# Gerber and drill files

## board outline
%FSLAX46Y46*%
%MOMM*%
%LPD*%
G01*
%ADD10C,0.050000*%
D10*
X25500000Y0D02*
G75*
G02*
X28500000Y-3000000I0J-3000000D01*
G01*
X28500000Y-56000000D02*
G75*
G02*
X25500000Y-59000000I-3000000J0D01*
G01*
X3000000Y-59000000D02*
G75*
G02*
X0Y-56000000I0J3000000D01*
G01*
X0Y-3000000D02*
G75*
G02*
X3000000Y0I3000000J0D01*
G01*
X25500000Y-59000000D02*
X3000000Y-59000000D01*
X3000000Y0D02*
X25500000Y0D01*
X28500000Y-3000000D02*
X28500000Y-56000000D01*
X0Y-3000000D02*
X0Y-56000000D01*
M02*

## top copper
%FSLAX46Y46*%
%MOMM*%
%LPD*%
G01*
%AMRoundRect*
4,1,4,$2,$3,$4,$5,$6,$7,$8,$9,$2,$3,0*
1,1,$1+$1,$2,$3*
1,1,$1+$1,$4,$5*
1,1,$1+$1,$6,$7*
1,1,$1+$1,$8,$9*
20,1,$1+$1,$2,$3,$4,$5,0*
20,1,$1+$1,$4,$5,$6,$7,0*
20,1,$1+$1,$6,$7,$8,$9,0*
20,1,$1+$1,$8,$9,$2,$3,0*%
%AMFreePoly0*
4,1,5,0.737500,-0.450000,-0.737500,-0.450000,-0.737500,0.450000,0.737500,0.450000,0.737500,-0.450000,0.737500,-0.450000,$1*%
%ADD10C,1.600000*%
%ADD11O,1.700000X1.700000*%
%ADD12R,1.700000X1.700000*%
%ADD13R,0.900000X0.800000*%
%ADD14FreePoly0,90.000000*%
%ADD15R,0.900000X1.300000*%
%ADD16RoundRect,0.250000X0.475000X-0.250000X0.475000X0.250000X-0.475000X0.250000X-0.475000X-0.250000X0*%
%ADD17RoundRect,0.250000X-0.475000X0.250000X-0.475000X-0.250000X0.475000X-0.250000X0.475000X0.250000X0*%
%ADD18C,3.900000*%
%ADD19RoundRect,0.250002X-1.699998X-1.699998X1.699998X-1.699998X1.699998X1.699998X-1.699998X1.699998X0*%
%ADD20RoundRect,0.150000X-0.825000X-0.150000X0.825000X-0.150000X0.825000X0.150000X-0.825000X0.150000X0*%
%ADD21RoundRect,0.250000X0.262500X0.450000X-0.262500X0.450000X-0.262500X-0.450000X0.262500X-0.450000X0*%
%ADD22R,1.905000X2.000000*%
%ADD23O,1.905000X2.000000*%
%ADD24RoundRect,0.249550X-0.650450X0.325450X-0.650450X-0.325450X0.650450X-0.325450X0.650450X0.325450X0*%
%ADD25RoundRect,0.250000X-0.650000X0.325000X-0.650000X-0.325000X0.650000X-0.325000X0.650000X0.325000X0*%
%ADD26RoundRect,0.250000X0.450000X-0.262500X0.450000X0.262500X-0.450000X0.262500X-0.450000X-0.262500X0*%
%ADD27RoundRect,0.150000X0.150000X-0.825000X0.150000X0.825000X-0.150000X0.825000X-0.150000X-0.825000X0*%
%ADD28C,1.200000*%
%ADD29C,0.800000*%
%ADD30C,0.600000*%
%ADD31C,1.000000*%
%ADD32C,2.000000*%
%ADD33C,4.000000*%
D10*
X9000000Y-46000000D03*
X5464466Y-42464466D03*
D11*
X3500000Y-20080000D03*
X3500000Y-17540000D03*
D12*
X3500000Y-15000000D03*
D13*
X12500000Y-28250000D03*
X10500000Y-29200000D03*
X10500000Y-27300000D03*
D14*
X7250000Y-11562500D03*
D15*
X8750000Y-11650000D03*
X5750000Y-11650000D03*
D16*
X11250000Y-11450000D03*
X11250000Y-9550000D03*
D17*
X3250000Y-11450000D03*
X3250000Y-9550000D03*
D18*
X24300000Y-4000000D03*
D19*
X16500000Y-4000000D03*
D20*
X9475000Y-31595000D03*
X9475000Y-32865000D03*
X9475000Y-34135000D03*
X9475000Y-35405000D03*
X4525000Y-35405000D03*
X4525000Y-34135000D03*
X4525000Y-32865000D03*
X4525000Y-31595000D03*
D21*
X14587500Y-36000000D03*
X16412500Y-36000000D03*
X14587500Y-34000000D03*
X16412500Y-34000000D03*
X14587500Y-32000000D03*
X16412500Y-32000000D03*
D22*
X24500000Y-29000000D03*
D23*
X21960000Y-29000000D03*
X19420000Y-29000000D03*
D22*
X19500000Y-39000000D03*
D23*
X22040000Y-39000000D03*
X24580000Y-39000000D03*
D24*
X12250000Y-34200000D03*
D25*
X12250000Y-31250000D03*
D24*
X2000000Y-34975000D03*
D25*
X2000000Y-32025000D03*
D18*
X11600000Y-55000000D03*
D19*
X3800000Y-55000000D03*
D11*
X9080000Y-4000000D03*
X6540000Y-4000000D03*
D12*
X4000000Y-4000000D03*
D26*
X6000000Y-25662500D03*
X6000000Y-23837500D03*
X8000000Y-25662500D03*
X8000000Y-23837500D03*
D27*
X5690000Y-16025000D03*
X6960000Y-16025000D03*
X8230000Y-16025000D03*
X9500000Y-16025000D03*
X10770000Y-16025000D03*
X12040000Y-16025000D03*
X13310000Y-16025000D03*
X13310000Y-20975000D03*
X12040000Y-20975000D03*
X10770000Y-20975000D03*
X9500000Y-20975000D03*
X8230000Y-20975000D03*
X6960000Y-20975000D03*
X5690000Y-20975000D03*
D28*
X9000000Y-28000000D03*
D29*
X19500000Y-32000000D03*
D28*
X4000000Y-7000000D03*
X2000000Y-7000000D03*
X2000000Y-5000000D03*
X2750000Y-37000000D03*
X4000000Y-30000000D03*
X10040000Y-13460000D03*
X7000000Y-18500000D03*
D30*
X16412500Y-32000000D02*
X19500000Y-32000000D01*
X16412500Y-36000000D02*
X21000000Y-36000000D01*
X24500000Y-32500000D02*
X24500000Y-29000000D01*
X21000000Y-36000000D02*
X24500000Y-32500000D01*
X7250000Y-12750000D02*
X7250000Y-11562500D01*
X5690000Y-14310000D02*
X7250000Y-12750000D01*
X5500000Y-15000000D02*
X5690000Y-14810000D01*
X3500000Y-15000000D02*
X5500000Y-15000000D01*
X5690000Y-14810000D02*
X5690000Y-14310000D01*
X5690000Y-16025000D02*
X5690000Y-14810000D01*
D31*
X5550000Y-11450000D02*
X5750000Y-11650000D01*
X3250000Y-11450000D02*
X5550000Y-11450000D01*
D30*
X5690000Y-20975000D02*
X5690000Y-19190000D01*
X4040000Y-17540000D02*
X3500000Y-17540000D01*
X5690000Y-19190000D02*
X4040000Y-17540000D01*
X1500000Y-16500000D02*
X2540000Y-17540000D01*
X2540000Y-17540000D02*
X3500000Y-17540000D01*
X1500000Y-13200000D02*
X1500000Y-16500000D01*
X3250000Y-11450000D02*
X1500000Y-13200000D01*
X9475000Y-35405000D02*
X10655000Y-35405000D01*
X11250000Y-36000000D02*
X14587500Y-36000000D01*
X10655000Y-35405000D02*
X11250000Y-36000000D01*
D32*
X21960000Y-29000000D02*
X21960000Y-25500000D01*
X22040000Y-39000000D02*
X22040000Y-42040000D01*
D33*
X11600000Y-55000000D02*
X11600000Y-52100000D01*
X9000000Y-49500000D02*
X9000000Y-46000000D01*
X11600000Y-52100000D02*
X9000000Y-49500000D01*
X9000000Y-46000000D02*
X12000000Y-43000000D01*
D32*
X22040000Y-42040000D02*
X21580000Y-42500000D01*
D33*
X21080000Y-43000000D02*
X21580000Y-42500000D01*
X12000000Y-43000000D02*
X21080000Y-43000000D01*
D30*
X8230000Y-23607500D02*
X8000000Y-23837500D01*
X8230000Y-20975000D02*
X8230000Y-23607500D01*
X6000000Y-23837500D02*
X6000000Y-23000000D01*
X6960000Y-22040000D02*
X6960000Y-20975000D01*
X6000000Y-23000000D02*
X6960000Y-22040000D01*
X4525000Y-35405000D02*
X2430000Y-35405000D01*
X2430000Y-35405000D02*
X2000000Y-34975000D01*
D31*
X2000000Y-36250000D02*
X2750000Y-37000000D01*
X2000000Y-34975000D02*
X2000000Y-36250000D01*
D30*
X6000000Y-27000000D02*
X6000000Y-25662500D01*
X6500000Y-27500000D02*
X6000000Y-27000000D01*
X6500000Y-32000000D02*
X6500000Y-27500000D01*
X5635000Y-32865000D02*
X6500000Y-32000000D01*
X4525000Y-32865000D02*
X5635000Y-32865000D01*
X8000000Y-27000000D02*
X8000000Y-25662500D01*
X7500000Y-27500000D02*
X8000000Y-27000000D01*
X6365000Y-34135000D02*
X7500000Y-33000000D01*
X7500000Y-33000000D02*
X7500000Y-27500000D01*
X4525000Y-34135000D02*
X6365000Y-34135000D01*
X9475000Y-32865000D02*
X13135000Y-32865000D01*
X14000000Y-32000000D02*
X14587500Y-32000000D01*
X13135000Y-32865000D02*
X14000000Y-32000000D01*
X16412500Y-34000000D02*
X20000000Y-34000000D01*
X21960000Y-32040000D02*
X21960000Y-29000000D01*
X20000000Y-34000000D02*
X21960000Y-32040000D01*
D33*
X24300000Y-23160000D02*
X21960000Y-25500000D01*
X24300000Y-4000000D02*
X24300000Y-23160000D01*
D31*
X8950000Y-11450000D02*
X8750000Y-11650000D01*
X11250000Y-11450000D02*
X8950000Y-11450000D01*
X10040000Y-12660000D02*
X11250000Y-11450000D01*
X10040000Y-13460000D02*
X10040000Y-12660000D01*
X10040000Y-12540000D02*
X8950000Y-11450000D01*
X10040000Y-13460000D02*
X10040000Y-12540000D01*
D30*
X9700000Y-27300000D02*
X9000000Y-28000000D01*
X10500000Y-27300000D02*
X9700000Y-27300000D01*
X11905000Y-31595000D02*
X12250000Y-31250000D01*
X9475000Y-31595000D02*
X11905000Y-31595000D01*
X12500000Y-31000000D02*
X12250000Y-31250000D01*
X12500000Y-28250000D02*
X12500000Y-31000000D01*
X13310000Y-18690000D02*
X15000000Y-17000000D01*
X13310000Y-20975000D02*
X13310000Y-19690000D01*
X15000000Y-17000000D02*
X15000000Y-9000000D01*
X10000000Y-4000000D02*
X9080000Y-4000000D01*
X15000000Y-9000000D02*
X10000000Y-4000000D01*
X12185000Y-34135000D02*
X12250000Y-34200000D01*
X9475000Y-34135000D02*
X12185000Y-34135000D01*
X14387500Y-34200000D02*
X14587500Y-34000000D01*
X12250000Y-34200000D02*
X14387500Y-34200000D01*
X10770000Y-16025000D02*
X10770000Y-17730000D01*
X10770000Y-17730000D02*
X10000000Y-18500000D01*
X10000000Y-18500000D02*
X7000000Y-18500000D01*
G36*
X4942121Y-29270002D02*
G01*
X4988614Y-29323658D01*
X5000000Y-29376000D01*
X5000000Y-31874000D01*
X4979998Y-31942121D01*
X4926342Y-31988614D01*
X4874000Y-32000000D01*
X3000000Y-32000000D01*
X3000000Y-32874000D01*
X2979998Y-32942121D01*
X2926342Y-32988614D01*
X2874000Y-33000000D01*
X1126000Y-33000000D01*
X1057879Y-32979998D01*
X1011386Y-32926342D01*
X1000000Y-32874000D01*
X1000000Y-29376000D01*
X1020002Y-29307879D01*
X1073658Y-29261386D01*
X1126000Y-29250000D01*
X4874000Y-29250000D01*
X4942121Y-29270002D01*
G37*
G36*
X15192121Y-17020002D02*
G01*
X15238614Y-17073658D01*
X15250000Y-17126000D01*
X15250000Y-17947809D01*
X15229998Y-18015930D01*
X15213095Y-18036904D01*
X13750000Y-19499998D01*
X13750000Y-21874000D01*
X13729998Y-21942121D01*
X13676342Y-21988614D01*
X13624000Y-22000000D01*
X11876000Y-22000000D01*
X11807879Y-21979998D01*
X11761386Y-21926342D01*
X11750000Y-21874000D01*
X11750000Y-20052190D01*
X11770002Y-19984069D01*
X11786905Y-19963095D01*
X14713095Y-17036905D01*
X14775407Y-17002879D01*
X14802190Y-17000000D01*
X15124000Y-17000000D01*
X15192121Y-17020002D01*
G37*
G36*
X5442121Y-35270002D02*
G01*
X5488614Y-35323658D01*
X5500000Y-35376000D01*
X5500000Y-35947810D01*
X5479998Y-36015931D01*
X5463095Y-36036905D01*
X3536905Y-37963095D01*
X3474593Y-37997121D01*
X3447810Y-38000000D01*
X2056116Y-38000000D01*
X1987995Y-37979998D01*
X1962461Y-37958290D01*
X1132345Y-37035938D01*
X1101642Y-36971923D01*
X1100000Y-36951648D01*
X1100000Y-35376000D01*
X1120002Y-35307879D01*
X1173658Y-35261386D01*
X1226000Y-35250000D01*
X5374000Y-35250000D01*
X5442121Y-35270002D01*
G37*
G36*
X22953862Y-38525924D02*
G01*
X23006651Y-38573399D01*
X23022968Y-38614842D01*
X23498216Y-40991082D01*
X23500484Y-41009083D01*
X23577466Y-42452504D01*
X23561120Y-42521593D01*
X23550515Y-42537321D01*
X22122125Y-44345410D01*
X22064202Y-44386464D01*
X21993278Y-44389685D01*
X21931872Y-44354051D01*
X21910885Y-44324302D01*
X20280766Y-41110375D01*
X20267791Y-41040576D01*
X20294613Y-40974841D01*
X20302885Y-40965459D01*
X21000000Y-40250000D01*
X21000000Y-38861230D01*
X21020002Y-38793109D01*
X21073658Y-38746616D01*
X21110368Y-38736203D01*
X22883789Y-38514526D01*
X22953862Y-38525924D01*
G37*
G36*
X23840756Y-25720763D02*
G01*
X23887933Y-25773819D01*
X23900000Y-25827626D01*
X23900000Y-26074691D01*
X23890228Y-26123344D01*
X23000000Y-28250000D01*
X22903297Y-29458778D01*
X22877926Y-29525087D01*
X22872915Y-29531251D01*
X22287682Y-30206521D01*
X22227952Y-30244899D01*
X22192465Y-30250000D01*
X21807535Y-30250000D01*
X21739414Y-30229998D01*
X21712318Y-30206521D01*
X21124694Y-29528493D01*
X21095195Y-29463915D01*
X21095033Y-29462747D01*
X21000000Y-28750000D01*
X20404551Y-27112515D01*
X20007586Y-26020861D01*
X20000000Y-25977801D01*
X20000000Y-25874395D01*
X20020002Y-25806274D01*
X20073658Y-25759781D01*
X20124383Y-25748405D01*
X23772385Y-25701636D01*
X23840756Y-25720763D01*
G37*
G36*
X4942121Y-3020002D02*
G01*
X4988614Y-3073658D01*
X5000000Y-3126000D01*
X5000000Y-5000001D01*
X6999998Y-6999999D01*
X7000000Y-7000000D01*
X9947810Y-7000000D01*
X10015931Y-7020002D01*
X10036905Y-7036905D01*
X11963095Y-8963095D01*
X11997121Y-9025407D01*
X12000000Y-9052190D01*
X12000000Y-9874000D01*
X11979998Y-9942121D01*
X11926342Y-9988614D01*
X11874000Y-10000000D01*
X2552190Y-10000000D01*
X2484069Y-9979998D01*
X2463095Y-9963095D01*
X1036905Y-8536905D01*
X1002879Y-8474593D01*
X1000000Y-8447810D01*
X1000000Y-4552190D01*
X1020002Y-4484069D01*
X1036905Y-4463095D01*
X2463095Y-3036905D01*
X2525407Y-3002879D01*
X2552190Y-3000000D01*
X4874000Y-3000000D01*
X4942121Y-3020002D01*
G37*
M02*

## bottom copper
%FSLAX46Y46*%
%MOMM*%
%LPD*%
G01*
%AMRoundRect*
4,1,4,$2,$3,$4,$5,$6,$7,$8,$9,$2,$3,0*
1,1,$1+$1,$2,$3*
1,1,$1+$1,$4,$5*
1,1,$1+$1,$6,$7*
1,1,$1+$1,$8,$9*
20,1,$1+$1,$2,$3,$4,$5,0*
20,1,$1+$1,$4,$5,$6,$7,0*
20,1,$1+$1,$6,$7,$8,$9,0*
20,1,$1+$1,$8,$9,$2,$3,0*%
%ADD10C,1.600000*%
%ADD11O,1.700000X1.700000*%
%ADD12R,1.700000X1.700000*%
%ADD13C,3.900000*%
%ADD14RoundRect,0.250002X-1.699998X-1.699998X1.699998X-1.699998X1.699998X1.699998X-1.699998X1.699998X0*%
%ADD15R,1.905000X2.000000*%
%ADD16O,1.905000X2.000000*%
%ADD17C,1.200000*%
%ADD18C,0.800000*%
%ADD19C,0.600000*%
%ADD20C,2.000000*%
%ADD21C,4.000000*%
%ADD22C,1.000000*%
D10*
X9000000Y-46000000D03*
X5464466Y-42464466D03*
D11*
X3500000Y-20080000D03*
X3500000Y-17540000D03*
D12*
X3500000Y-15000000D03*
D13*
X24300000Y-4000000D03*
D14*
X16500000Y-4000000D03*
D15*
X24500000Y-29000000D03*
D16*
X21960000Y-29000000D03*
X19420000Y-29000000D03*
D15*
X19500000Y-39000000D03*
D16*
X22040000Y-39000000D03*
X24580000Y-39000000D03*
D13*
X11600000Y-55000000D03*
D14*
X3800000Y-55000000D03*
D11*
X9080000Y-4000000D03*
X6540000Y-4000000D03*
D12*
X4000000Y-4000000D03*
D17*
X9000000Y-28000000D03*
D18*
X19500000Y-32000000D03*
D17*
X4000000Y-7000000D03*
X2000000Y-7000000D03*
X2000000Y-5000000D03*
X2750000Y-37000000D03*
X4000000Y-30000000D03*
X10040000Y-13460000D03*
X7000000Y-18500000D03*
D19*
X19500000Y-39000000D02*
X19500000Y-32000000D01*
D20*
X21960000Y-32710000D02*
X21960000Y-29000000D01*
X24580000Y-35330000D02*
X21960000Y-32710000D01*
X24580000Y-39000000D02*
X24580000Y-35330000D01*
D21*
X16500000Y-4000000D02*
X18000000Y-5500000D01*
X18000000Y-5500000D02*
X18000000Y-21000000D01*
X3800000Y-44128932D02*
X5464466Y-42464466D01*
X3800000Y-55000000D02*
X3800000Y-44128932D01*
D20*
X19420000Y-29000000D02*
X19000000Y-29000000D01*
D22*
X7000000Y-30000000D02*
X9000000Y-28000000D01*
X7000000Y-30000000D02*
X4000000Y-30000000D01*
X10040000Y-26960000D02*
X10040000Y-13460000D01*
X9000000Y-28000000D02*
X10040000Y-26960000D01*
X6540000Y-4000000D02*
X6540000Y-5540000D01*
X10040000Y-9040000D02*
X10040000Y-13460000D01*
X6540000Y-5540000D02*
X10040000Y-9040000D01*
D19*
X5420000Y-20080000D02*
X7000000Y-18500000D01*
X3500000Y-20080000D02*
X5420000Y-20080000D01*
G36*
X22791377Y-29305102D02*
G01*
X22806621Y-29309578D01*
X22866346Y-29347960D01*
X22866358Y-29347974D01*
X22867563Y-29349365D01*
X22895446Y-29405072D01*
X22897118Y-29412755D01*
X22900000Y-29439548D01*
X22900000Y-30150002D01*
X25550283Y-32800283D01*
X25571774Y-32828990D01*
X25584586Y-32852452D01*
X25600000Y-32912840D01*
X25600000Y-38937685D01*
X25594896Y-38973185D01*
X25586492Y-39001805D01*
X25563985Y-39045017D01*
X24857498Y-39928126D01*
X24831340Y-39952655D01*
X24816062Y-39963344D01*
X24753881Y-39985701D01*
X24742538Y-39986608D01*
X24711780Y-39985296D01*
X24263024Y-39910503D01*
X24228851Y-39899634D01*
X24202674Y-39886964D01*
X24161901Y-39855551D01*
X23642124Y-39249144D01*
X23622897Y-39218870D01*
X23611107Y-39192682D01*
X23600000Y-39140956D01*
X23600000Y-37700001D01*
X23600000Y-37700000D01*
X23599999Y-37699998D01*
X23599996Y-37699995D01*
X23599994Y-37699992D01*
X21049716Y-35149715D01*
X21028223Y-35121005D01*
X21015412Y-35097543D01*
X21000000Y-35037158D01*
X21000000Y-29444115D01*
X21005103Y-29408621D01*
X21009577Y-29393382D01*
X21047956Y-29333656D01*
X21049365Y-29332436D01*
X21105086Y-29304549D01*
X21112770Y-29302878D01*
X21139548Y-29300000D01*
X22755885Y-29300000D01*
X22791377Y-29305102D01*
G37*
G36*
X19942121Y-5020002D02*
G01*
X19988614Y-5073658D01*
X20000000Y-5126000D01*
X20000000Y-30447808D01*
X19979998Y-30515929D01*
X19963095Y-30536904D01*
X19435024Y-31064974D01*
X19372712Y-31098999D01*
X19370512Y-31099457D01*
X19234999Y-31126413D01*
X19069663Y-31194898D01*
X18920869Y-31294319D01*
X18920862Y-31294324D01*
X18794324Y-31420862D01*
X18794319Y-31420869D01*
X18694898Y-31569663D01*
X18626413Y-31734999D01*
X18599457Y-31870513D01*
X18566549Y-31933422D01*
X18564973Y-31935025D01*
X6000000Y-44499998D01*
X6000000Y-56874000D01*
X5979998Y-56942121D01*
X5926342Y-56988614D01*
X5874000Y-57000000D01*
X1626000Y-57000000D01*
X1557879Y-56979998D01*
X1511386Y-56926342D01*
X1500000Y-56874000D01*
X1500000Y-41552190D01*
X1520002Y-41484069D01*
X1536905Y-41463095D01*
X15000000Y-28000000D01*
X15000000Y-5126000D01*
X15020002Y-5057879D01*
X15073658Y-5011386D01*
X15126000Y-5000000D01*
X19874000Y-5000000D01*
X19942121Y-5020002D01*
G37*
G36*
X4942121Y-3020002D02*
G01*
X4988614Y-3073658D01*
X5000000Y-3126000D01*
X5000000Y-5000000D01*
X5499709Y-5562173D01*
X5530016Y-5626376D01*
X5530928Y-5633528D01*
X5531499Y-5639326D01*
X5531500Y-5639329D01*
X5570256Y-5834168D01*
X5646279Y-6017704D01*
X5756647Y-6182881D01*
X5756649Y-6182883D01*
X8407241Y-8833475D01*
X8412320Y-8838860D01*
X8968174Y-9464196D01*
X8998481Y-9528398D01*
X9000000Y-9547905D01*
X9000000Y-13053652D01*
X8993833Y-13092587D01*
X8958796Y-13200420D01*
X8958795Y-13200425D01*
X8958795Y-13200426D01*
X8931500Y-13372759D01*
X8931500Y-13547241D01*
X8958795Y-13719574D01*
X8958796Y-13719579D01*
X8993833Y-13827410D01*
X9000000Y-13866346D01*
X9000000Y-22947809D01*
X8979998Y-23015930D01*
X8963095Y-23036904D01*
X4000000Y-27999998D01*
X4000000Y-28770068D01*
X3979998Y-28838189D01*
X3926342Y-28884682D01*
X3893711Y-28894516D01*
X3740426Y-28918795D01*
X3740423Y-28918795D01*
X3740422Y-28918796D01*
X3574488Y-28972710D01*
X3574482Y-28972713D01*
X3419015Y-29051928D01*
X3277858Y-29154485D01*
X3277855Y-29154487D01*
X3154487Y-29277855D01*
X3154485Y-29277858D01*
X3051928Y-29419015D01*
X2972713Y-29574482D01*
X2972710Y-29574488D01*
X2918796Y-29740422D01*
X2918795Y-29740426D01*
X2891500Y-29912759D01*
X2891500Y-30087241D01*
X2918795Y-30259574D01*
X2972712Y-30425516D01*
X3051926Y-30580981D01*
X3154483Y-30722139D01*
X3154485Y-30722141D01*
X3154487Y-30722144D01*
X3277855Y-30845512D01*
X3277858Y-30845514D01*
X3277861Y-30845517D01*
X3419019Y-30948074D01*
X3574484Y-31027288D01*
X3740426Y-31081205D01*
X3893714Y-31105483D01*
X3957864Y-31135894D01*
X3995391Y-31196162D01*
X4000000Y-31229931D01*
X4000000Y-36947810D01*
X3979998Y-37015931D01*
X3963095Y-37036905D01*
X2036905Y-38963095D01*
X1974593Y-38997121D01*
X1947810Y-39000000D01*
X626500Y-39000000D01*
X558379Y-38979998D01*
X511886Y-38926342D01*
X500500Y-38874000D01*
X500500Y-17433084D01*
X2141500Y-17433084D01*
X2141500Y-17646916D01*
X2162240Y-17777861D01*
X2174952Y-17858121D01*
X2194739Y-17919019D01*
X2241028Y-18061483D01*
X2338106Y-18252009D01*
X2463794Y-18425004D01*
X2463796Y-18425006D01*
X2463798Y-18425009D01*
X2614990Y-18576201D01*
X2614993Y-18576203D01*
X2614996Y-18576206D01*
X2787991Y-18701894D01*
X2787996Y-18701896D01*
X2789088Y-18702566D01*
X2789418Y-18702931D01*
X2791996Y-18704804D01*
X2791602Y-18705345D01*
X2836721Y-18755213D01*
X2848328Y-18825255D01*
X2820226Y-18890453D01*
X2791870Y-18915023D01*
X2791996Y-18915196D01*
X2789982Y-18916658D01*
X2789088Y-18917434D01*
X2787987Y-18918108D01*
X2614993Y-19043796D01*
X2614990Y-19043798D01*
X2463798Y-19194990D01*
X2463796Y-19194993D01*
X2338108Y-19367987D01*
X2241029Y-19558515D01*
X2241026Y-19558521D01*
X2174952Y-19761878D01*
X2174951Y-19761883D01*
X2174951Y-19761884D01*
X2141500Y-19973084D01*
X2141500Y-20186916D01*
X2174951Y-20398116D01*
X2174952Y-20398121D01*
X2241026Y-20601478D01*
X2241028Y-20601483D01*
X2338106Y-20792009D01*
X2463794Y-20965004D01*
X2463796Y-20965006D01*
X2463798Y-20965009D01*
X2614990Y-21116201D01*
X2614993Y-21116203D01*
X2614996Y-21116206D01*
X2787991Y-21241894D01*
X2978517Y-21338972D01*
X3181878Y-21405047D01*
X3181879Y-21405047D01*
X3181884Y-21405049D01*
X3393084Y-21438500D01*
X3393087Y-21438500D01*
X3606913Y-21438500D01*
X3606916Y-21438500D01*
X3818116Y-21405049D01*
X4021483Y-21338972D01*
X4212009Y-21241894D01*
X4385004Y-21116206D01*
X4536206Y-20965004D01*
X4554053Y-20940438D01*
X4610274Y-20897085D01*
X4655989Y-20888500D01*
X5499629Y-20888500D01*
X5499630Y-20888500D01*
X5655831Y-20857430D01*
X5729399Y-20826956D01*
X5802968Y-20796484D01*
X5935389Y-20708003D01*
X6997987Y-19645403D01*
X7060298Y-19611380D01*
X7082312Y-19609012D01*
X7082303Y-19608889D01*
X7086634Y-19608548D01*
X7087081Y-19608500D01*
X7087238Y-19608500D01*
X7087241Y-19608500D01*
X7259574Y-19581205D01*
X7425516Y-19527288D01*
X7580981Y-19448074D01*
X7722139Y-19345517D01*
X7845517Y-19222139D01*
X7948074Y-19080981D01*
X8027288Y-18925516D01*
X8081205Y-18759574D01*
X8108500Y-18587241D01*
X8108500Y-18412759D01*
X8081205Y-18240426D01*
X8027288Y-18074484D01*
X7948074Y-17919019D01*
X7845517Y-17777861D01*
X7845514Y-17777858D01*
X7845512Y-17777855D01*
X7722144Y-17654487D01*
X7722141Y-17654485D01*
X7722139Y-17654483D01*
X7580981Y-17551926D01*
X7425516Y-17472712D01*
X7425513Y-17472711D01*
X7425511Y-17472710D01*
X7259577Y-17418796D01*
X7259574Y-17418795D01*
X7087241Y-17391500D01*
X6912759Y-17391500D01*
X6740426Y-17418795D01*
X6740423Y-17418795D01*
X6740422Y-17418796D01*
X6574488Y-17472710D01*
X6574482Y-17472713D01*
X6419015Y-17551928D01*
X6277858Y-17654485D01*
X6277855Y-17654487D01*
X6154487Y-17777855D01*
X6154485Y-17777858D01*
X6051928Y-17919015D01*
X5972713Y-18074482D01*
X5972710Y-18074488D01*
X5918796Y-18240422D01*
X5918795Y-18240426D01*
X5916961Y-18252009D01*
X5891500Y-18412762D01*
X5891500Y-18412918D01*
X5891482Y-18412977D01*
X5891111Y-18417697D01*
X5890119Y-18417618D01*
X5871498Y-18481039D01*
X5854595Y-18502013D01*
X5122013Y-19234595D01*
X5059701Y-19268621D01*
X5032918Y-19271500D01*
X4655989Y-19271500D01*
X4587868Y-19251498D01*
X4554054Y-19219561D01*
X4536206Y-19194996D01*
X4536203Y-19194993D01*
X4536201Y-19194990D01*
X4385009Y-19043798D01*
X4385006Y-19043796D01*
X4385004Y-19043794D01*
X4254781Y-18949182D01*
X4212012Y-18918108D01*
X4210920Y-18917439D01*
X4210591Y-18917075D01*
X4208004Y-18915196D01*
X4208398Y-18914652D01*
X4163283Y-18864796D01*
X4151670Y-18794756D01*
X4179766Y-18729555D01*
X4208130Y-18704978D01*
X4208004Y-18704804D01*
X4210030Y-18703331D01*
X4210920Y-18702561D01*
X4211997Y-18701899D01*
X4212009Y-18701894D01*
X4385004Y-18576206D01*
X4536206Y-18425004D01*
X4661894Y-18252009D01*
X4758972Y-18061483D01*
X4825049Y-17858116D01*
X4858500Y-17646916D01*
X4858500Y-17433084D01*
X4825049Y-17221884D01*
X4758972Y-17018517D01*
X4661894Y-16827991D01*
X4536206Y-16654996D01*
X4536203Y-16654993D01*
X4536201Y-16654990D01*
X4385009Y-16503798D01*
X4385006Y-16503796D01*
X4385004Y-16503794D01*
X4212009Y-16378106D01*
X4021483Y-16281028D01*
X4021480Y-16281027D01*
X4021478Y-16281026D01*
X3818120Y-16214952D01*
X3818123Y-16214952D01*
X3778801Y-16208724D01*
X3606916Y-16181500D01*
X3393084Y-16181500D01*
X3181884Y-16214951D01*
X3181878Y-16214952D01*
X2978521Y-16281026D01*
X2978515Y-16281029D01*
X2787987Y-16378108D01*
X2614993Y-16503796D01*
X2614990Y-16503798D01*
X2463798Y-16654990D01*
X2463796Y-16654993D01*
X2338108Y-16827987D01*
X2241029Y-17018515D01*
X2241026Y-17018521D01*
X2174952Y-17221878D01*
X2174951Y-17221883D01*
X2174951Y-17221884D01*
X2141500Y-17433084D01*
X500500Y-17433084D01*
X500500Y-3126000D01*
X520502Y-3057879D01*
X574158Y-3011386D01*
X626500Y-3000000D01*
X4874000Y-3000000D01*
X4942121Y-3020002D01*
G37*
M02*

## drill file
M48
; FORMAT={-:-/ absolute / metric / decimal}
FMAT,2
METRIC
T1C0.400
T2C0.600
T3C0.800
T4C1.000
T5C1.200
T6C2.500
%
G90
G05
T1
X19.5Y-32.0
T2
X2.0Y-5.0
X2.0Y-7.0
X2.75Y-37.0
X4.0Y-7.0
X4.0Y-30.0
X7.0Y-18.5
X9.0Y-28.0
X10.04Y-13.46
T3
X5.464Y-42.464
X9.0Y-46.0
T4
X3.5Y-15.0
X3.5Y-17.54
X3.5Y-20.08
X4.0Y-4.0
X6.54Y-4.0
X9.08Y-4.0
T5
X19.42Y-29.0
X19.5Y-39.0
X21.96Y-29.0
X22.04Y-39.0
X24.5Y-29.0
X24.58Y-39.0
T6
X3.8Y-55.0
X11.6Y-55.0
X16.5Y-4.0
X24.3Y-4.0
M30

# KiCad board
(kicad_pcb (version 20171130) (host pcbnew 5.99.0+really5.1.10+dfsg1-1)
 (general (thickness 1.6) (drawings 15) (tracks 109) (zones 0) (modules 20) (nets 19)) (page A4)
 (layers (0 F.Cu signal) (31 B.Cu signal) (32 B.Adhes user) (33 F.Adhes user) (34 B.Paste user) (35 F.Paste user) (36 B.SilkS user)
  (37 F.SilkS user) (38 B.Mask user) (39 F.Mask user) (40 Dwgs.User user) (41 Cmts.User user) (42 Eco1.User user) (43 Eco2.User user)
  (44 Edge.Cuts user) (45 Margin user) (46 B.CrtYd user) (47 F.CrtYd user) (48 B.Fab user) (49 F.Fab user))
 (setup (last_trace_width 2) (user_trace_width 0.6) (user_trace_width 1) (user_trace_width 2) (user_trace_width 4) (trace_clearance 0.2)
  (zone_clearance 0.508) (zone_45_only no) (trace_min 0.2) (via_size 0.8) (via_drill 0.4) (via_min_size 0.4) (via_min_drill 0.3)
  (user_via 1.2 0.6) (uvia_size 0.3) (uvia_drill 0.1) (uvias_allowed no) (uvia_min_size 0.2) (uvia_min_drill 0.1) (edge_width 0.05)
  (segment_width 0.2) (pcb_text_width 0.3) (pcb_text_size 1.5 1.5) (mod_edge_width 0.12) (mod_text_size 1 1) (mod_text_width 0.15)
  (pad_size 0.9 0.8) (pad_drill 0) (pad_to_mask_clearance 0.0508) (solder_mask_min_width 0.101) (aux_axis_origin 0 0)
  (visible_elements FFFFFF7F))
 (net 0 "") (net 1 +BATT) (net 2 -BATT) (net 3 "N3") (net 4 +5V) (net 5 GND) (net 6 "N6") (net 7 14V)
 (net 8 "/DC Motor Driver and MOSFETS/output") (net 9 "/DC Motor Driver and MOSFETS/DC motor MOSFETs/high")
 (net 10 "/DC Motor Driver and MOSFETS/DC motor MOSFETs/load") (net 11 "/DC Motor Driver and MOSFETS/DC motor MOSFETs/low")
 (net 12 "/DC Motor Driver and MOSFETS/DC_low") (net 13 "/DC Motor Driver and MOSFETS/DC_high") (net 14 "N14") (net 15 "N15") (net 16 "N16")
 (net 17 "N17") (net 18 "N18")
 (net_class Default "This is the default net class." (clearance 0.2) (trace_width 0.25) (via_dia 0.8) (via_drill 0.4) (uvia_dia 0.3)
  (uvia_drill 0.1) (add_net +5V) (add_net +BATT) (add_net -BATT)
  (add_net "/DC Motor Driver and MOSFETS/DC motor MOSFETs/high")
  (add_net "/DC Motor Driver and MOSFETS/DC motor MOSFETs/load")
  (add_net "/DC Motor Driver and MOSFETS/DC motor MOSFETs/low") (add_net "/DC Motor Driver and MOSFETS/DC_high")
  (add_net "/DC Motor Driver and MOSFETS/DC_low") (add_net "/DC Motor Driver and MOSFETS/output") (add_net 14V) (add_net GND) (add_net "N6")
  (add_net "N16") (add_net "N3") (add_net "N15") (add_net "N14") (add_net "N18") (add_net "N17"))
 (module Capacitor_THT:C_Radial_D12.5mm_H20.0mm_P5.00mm (layer F.Cu) (at 9 46 135)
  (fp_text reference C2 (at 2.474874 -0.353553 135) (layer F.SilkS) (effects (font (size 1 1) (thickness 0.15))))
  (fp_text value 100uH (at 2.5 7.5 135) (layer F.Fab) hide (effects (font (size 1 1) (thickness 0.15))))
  (pad 1 thru_hole circle (at 0 0 135) (size 1.6 1.6) (drill 0.8) (layers *.Cu *.Mask) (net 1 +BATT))
  (pad 2 thru_hole circle (at 5 0 135) (size 1.6 1.6) (drill 0.8) (layers *.Cu *.Mask) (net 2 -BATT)))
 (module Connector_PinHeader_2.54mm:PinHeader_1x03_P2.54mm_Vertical (layer B.Cu) (at 3.5 15 180)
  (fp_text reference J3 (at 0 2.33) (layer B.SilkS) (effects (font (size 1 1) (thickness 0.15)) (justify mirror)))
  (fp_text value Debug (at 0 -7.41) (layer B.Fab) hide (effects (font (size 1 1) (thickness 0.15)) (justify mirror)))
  (pad 3 thru_hole oval (at 0 -5.08 180) (size 1.7 1.7) (drill 1) (layers *.Cu *.Mask) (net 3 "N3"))
  (pad 2 thru_hole oval (at 0 -2.54 180) (size 1.7 1.7) (drill 1) (layers *.Cu *.Mask) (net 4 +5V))
  (pad 1 thru_hole rect (at 0 0 180) (size 1.7 1.7) (drill 1) (layers *.Cu *.Mask) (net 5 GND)))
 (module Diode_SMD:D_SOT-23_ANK (layer F.Cu) (at 11.5 28.25)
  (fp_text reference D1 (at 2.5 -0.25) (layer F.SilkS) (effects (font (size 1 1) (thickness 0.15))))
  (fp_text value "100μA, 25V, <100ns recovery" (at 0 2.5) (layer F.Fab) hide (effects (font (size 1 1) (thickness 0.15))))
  (pad 1 smd rect (at 1 0) (size 0.9 0.8) (layers F.Cu F.Paste F.Mask) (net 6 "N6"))
  (pad "" smd rect (at -1 0.95) (size 0.9 0.8) (layers F.Cu F.Paste F.Mask))
  (pad 2 smd rect (at -1 -0.95) (size 0.9 0.8) (layers F.Cu F.Paste F.Mask) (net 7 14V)))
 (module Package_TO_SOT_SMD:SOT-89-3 (layer F.Cu) (at 7.25 10 90)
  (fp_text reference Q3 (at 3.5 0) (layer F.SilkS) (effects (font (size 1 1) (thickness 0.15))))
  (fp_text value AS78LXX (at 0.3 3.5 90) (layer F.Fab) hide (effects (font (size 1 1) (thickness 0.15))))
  (pad 2 smd custom (at -1.5625 0 90) (size 1.475 0.9) (layers F.Cu F.Paste F.Mask) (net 5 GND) (zone_connect 2)
   (options (clearance outline) (anchor rect)) (primitives))
  (pad 3 smd rect (at -1.65 1.5 90) (size 1.3 0.9) (layers F.Cu F.Paste F.Mask) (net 7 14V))
  (pad 1 smd rect (at -1.65 -1.5 90) (size 1.3 0.9) (layers F.Cu F.Paste F.Mask) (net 4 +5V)))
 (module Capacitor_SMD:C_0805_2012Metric (layer F.Cu) (at 11.25 10.5 90)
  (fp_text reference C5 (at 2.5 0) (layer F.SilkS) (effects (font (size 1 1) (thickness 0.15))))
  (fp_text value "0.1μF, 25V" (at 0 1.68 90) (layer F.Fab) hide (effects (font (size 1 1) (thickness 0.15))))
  (pad 1 smd roundrect (at -0.95 0 90) (size 1 1.45) (layers F.Cu F.Paste F.Mask) (roundrect_rratio 0.25) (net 7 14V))
  (pad 2 smd roundrect (at 0.95 0 90) (size 1 1.45) (layers F.Cu F.Paste F.Mask) (roundrect_rratio 0.25) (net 5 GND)))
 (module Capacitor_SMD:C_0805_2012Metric (layer F.Cu) (at 3.25 10.5 270)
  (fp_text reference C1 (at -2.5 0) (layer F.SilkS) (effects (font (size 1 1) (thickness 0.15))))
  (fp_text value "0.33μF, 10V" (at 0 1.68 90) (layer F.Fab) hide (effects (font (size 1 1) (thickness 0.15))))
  (pad 2 smd roundrect (at 0.95 0 270) (size 1 1.45) (layers F.Cu F.Paste F.Mask) (roundrect_rratio 0.25) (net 4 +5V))
  (pad 1 smd roundrect (at -0.95 0 270) (size 1 1.45) (layers F.Cu F.Paste F.Mask) (roundrect_rratio 0.25) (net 5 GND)))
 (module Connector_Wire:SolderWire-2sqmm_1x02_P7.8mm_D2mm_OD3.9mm (layer F.Cu) (at 16.5 4)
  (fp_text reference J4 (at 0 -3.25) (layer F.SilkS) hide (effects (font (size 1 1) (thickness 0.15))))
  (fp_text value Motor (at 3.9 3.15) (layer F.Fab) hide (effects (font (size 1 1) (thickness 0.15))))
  (pad 2 thru_hole circle (at 7.8 0) (size 3.9 3.9) (drill 2.5) (layers *.Cu *.Mask) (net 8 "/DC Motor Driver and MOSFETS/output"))
  (pad 1 thru_hole roundrect (at 0 0) (size 3.9 3.9) (drill 2.5) (layers *.Cu *.Mask) (roundrect_rratio 0.06410299999999999) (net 2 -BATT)))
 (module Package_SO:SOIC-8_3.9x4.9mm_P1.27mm (layer F.Cu) (at 7 33.5)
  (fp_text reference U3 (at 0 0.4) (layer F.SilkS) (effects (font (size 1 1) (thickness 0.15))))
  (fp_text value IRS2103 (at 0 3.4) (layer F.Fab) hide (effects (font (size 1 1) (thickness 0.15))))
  (pad 8 smd roundrect (at 2.475 -1.905) (size 1.95 0.6) (layers F.Cu F.Paste F.Mask) (roundrect_rratio 0.25) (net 6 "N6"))
  (pad 7 smd roundrect (at 2.475 -0.635) (size 1.95 0.6) (layers F.Cu F.Paste F.Mask) (roundrect_rratio 0.25)
   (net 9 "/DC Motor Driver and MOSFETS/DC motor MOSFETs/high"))
  (pad 6 smd roundrect (at 2.475 0.635) (size 1.95 0.6) (layers F.Cu F.Paste F.Mask) (roundrect_rratio 0.25)
   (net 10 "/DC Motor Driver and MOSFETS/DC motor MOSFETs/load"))
  (pad 5 smd roundrect (at 2.475 1.905) (size 1.95 0.6) (layers F.Cu F.Paste F.Mask) (roundrect_rratio 0.25)
   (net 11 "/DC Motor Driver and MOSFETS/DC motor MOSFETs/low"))
  (pad 4 smd roundrect (at -2.475 1.905) (size 1.95 0.6) (layers F.Cu F.Paste F.Mask) (roundrect_rratio 0.25) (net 5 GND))
  (pad 3 smd roundrect (at -2.475 0.635) (size 1.95 0.6) (layers F.Cu F.Paste F.Mask) (roundrect_rratio 0.25)
   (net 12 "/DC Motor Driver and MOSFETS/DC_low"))
  (pad 2 smd roundrect (at -2.475 -0.635) (size 1.95 0.6) (layers F.Cu F.Paste F.Mask) (roundrect_rratio 0.25)
   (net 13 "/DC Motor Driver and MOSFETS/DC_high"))
  (pad 1 smd roundrect (at -2.475 -1.905) (size 1.95 0.6) (layers F.Cu F.Paste F.Mask) (roundrect_rratio 0.25) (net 7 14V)))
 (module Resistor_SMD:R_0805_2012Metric (layer F.Cu) (at 15.5 36 180)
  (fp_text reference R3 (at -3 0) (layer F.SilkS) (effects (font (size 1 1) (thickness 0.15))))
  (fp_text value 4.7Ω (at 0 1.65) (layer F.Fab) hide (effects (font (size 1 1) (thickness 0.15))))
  (pad 2 smd roundrect (at 0.9125 0 180) (size 1.025 1.4) (layers F.Cu F.Paste F.Mask) (roundrect_rratio 0.243902)
   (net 11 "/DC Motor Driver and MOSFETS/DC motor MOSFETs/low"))
  (pad 1 smd roundrect (at -0.9125 0 180) (size 1.025 1.4) (layers F.Cu F.Paste F.Mask) (roundrect_rratio 0.243902) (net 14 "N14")))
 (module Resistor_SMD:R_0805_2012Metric (layer F.Cu) (at 15.5 34 180)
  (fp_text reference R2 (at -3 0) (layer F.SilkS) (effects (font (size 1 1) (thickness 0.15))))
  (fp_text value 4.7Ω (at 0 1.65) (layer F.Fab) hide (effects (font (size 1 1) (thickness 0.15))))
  (pad 2 smd roundrect (at 0.9125 0 180) (size 1.025 1.4) (layers F.Cu F.Paste F.Mask) (roundrect_rratio 0.243902)
   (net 10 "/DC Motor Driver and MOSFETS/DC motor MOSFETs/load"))
  (pad 1 smd roundrect (at -0.9125 0 180) (size 1.025 1.4) (layers F.Cu F.Paste F.Mask) (roundrect_rratio 0.243902)
   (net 8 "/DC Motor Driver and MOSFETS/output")))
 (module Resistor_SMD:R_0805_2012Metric (layer F.Cu) (at 15.5 32 180)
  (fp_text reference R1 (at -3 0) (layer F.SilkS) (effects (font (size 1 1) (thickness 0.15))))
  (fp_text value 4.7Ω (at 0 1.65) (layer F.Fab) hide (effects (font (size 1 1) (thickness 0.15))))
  (pad 2 smd roundrect (at 0.9125 0 180) (size 1.025 1.4) (layers F.Cu F.Paste F.Mask) (roundrect_rratio 0.243902)
   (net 9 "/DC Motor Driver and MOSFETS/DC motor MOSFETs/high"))
  (pad 1 smd roundrect (at -0.9125 0 180) (size 1.025 1.4) (layers F.Cu F.Paste F.Mask) (roundrect_rratio 0.243902) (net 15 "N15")))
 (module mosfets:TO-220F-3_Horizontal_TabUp (layer F.Cu) (at 24.5 29 180)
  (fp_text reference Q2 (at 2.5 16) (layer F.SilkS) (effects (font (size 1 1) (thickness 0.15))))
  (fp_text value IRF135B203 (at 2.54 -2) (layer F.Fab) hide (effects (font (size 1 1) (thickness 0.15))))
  (pad 1 thru_hole rect (at 0 0 180) (size 1.905 2) (drill 1.2) (layers *.Cu *.Mask) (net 14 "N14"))
  (pad 2 thru_hole oval (at 2.54 0 180) (size 1.905 2) (drill 1.2) (layers *.Cu *.Mask) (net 8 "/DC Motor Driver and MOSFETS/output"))
  (pad 3 thru_hole oval (at 5.08 0 180) (size 1.905 2) (drill 1.2) (layers *.Cu *.Mask) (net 2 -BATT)))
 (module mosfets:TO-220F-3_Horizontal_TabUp (layer F.Cu) (at 19.5 39)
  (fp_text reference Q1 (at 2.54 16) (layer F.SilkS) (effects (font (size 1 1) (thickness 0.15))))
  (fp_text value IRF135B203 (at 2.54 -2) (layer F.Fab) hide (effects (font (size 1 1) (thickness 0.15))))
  (pad 1 thru_hole rect (at 0 0) (size 1.905 2) (drill 1.2) (layers *.Cu *.Mask) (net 15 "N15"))
  (pad 2 thru_hole oval (at 2.54 0) (size 1.905 2) (drill 1.2) (layers *.Cu *.Mask) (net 1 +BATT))
  (pad 3 thru_hole oval (at 5.08 0) (size 1.905 2) (drill 1.2) (layers *.Cu *.Mask) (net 8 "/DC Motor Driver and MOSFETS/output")))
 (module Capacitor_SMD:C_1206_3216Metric (layer F.Cu) (at 12.25 32.725 270)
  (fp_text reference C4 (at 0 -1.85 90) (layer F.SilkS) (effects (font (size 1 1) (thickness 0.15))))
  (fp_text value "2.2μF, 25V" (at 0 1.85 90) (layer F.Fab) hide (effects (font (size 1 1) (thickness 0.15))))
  (pad 2 smd roundrect (at 1.475 0 270) (size 1.15 1.8) (layers F.Cu F.Paste F.Mask) (roundrect_rratio 0.217)
   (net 10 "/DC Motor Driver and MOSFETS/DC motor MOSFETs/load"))
  (pad 1 smd roundrect (at -1.475 0 270) (size 1.15 1.8) (layers F.Cu F.Paste F.Mask) (roundrect_rratio 0.217391) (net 6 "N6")))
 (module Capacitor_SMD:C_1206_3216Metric (layer F.Cu) (at 2 33.5 270)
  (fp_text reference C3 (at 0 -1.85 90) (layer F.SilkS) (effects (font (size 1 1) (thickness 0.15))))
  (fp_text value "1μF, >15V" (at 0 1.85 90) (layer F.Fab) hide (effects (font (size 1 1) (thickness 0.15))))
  (pad 2 smd roundrect (at 1.475 0 270) (size 1.15 1.8) (layers F.Cu F.Paste F.Mask) (roundrect_rratio 0.217) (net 5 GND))
  (pad 1 smd roundrect (at -1.475 0 270) (size 1.15 1.8) (layers F.Cu F.Paste F.Mask) (roundrect_rratio 0.217391) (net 7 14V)))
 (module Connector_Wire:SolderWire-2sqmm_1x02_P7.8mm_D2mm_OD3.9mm (layer F.Cu) (at 3.8 55)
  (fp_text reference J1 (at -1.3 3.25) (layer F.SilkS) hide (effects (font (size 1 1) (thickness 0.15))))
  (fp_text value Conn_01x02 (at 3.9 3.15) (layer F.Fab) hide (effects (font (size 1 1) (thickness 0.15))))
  (pad 2 thru_hole circle (at 7.8 0) (size 3.9 3.9) (drill 2.5) (layers *.Cu *.Mask) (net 1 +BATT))
  (pad 1 thru_hole roundrect (at 0 0) (size 3.9 3.9) (drill 2.5) (layers *.Cu *.Mask) (roundrect_rratio 0.06410299999999999) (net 2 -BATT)))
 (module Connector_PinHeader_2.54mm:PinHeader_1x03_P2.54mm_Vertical (layer F.Cu) (at 4 4 90)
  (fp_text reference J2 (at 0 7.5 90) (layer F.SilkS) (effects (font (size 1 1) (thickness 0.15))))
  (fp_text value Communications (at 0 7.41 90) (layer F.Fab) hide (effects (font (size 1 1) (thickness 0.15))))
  (pad 3 thru_hole oval (at 0 5.08 90) (size 1.7 1.7) (drill 1) (layers *.Cu *.Mask) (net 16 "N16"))
  (pad 2 thru_hole oval (at 0 2.54 90) (size 1.7 1.7) (drill 1) (layers *.Cu *.Mask) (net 7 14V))
  (pad 1 thru_hole rect (at 0 0 90) (size 1.7 1.7) (drill 1) (layers *.Cu *.Mask) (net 5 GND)))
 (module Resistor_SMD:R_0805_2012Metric (layer F.Cu) (at 6 24.75 90)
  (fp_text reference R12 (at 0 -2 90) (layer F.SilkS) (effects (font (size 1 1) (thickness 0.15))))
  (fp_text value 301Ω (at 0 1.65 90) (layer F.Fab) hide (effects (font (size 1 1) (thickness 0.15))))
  (pad 1 smd roundrect (at -0.9125 0 90) (size 1.025 1.4) (layers F.Cu F.Paste F.Mask) (roundrect_rratio 0.243902)
   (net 13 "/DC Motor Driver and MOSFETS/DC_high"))
  (pad 2 smd roundrect (at 0.9125 0 90) (size 1.025 1.4) (layers F.Cu F.Paste F.Mask) (roundrect_rratio 0.243902) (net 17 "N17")))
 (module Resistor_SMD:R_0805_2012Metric (layer F.Cu) (at 8 24.75 90)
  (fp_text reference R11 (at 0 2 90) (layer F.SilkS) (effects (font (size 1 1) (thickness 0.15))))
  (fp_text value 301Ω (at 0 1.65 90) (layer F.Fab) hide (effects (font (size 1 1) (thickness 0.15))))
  (pad 1 smd roundrect (at -0.9125 0 90) (size 1.025 1.4) (layers F.Cu F.Paste F.Mask) (roundrect_rratio 0.243902)
   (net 12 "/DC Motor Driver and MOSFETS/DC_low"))
  (pad 2 smd roundrect (at 0.9125 0 90) (size 1.025 1.4) (layers F.Cu F.Paste F.Mask) (roundrect_rratio 0.243902) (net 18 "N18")))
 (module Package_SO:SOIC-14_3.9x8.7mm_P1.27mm (layer F.Cu) (at 9.5 18.5 90)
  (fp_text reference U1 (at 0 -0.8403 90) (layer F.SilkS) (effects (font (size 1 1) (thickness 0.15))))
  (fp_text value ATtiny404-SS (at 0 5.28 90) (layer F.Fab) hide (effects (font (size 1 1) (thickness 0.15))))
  (pad 14 smd roundrect (at 2.475 -3.81 90) (size 1.95 0.6) (layers F.Cu F.Paste F.Mask) (roundrect_rratio 0.25) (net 5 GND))
  (pad 13 smd roundrect (at 2.475 -2.54 90) (size 1.95 0.6) (layers F.Cu F.Paste F.Mask) (roundrect_rratio 0.25))
  (pad 12 smd roundrect (at 2.475 -1.27 90) (size 1.95 0.6) (layers F.Cu F.Paste F.Mask) (roundrect_rratio 0.25))
  (pad 11 smd roundrect (at 2.475 0 90) (size 1.95 0.6) (layers F.Cu F.Paste F.Mask) (roundrect_rratio 0.25))
  (pad 10 smd roundrect (at 2.475 1.27 90) (size 1.95 0.6) (layers F.Cu F.Paste F.Mask) (roundrect_rratio 0.25) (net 3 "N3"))
  (pad 9 smd roundrect (at 2.475 2.54 90) (size 1.95 0.6) (layers F.Cu F.Paste F.Mask) (roundrect_rratio 0.25))
  (pad 8 smd roundrect (at 2.475 3.81 90) (size 1.95 0.6) (layers F.Cu F.Paste F.Mask) (roundrect_rratio 0.25))
  (pad 7 smd roundrect (at -2.475 3.81 90) (size 1.95 0.6) (layers F.Cu F.Paste F.Mask) (roundrect_rratio 0.25) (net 16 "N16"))
  (pad 6 smd roundrect (at -2.475 2.54 90) (size 1.95 0.6) (layers F.Cu F.Paste F.Mask) (roundrect_rratio 0.25) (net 16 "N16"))
  (pad 5 smd roundrect (at -2.475 1.27 90) (size 1.95 0.6) (layers F.Cu F.Paste F.Mask) (roundrect_rratio 0.25))
  (pad 4 smd roundrect (at -2.475 0 90) (size 1.95 0.6) (layers F.Cu F.Paste F.Mask) (roundrect_rratio 0.25))
  (pad 3 smd roundrect (at -2.475 -1.27 90) (size 1.95 0.6) (layers F.Cu F.Paste F.Mask) (roundrect_rratio 0.25) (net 18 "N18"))
  (pad 2 smd roundrect (at -2.475 -2.54 90) (size 1.95 0.6) (layers F.Cu F.Paste F.Mask) (roundrect_rratio 0.25) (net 17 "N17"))
  (pad 1 smd roundrect (at -2.475 -3.81 90) (size 1.95 0.6) (layers F.Cu F.Paste F.Mask) (roundrect_rratio 0.25) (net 4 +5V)))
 (gr_arc (start 25.5 3) (end 28.5 3) (angle -90) (layer Edge.Cuts) (width 0.05))
 (gr_arc (start 25.5 56) (end 25.5 59) (angle -90) (layer Edge.Cuts) (width 0.05))
 (gr_arc (start 3 56) (end 0 56) (angle -90) (layer Edge.Cuts) (width 0.05))
 (gr_arc (start 3 3) (end 3 0) (angle -90) (layer Edge.Cuts) (width 0.05))
 (gr_line (start 25.5 59) (end 3 59) (layer Edge.Cuts) (width 0.05))
 (gr_line (start 3 0) (end 25.5 0) (layer Edge.Cuts) (width 0.05))
 (gr_line (start 28.5 3) (end 28.5 56) (layer Edge.Cuts) (width 0.05))
 (gr_line (start 0 3) (end 0 56) (layer Edge.Cuts) (width 0.05))
 (via (at 9 28) (size 1.2) (drill 0.6) (layers F.Cu B.Cu) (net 7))
 (via (at 19.5 32) (size 0.8) (drill 0.4) (layers F.Cu B.Cu) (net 15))
 (segment (start 19.5 39) (end 19.5 32) (width 0.6) (layer B.Cu) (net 15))
 (segment (start 16.4125 32) (end 19.5 32) (width 0.6) (layer F.Cu) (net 15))
 (segment (start 16.4125 36) (end 21 36) (width 0.6) (layer F.Cu) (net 14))
 (segment (start 24.5 32.5) (end 24.5 29) (width 0.6) (layer F.Cu) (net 14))
 (segment (start 21 36) (end 24.5 32.5) (width 0.6) (layer F.Cu) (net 14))
 (via (at 4 7) (size 1.2) (drill 0.6) (layers F.Cu B.Cu) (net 5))
 (segment (start 7.25 12.75) (end 7.25 11.5625) (width 0.6) (layer F.Cu) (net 5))
 (segment (start 5.69 14.31) (end 7.25 12.75) (width 0.6) (layer F.Cu) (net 5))
 (segment (start 5.5 15) (end 5.69 14.81) (width 0.6) (layer F.Cu) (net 5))
 (segment (start 3.5 15) (end 5.5 15) (width 0.6) (layer F.Cu) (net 5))
 (segment (start 5.69 14.81) (end 5.69 14.31) (width 0.6) (layer F.Cu) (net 5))
 (segment (start 5.69 16.025) (end 5.69 14.81) (width 0.6) (layer F.Cu) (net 5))
 (segment (start 5.55 11.45) (end 5.75 11.65) (width 1) (layer F.Cu) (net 4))
 (segment (start 3.25 11.45) (end 5.55 11.45) (width 1) (layer F.Cu) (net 4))
 (segment (start 5.69 20.975) (end 5.69 19.19) (width 0.6) (layer F.Cu) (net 4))
 (segment (start 4.04 17.54) (end 3.5 17.54) (width 0.6) (layer F.Cu) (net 4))
 (segment (start 5.69 19.19) (end 4.04 17.54) (width 0.6) (layer F.Cu) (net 4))
 (segment (start 1.5 16.5) (end 2.54 17.54) (width 0.6) (layer F.Cu) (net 4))
 (segment (start 2.54 17.54) (end 3.5 17.54) (width 0.6) (layer F.Cu) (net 4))
 (segment (start 1.5 13.2) (end 1.5 16.5) (width 0.6) (layer F.Cu) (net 4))
 (segment (start 3.25 11.45) (end 1.5 13.2) (width 0.6) (layer F.Cu) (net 4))
 (segment (start 9.475 35.405) (end 10.655 35.405) (width 0.6) (layer F.Cu) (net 11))
 (segment (start 11.25 36) (end 14.5875 36) (width 0.6) (layer F.Cu) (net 11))
 (segment (start 10.655 35.405) (end 11.25 36) (width 0.6) (layer F.Cu) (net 11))
 (segment (start 21.96 32.71) (end 21.96 29) (width 2) (layer B.Cu) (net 8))
 (segment (start 24.58 35.33) (end 21.96 32.71) (width 2) (layer B.Cu) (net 8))
 (segment (start 21.96 29) (end 21.96 25.5) (width 2) (layer F.Cu) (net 8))
 (segment (start 24.58 39) (end 24.58 35.33) (width 2) (layer B.Cu) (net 8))
 (segment (start 22.04 39) (end 22.04 42.04) (width 2) (layer F.Cu) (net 1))
 (segment (start 11.6 55) (end 11.6 52.1) (width 4) (layer F.Cu) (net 1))
 (segment (start 9 49.5) (end 9 46) (width 4) (layer F.Cu) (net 1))
 (segment (start 11.6 52.1) (end 9 49.5) (width 4) (layer F.Cu) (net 1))
 (segment (start 9 46) (end 12 43) (width 4) (layer F.Cu) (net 1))
 (segment (start 22.04 42.04) (end 21.58 42.5) (width 2) (layer F.Cu) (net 1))
 (segment (start 21.08 43) (end 21.58 42.5) (width 4) (layer F.Cu) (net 1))
 (segment (start 12 43) (end 21.08 43) (width 4) (layer F.Cu) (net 1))
 (segment (start 8.23 23.6075) (end 8 23.8375) (width 0.6) (layer F.Cu) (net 18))
 (segment (start 8.23 20.975) (end 8.23 23.6075) (width 0.6) (layer F.Cu) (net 18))
 (segment (start 6 23.8375) (end 6 23) (width 0.6) (layer F.Cu) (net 17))
 (segment (start 6.96 22.04) (end 6.96 20.975) (width 0.6) (layer F.Cu) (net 17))
 (segment (start 6 23) (end 6.96 22.04) (width 0.6) (layer F.Cu) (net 17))
 (via (at 2 7) (size 1.2) (drill 0.6) (layers F.Cu B.Cu) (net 5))
 (via (at 2 5) (size 1.2) (drill 0.6) (layers F.Cu B.Cu) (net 5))
 (segment (start 4.525 35.405) (end 2.43 35.405) (width 0.6) (layer F.Cu) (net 5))
 (segment (start 2.43 35.405) (end 2 34.975) (width 0.6) (layer F.Cu) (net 5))
 (segment (start 2 36.25) (end 2.75 37) (width 1) (layer F.Cu) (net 5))
 (via (at 2.75 37) (size 1.2) (drill 0.6) (layers F.Cu B.Cu) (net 5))
 (segment (start 2 34.975) (end 2 36.25) (width 1) (layer F.Cu) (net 5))
 (segment (start 6 27) (end 6 25.6625) (width 0.6) (layer F.Cu) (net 13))
 (segment (start 6.5 27.5) (end 6 27) (width 0.6) (layer F.Cu) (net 13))
 (segment (start 6.5 32) (end 6.5 27.5) (width 0.6) (layer F.Cu) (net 13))
 (segment (start 5.635 32.865) (end 6.5 32) (width 0.6) (layer F.Cu) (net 13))
 (segment (start 4.525 32.865) (end 5.635 32.865) (width 0.6) (layer F.Cu) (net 13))
 (segment (start 8 27) (end 8 25.6625) (width 0.6) (layer F.Cu) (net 12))
 (segment (start 7.5 27.5) (end 8 27) (width 0.6) (layer F.Cu) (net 12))
 (segment (start 6.365 34.135) (end 7.5 33) (width 0.6) (layer F.Cu) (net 12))
 (segment (start 7.5 33) (end 7.5 27.5) (width 0.6) (layer F.Cu) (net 12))
 (segment (start 4.525 34.135) (end 6.365 34.135) (width 0.6) (layer F.Cu) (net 12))
 (segment (start 9.475 32.865) (end 13.135 32.865) (width 0.6) (layer F.Cu) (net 9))
 (segment (start 14 32) (end 14.5875 32) (width 0.6) (layer F.Cu) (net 9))
 (segment (start 13.135 32.865) (end 14 32) (width 0.6) (layer F.Cu) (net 9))
 (segment (start 16.4125 34) (end 20 34) (width 0.6) (layer F.Cu) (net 8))
 (segment (start 21.96 32.04) (end 21.96 29) (width 0.6) (layer F.Cu) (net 8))
 (segment (start 20 34) (end 21.96 32.04) (width 0.6) (layer F.Cu) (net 8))
 (segment (start 24.3 23.16) (end 21.96 25.5) (width 4) (layer F.Cu) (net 8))
 (segment (start 24.3 4) (end 24.3 23.16) (width 4) (layer F.Cu) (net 8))
 (segment (start 16.5 4) (end 18 5.5) (width 4) (layer B.Cu) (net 2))
 (segment (start 18 5.5) (end 18 21) (width 4) (layer B.Cu) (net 2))
 (segment (start 3.8 44.128932) (end 5.464466 42.464466) (width 4) (layer B.Cu) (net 2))
 (segment (start 3.8 55) (end 3.8 44.128932) (width 4) (layer B.Cu) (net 2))
 (segment (start 19.42 29) (end 19 29) (width 2) (layer B.Cu) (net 2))
 (segment (start 8.95 11.45) (end 8.75 11.65) (width 1) (layer F.Cu) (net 7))
 (segment (start 11.25 11.45) (end 8.95 11.45) (width 1) (layer F.Cu) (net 7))
 (via (at 4 30) (size 1.2) (drill 0.6) (layers F.Cu B.Cu) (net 7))
 (via (at 10.04 13.46) (size 1.2) (drill 0.6) (layers F.Cu B.Cu) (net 7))
 (segment (start 10.04 12.66) (end 11.25 11.45) (width 1) (layer F.Cu) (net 7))
 (segment (start 10.04 13.46) (end 10.04 12.66) (width 1) (layer F.Cu) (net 7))
 (segment (start 10.04 12.54) (end 8.95 11.45) (width 1) (layer F.Cu) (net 7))
 (segment (start 10.04 13.46) (end 10.04 12.54) (width 1) (layer F.Cu) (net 7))
 (segment (start 9.7 27.3) (end 9 28) (width 0.6) (layer F.Cu) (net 7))
 (segment (start 10.5 27.3) (end 9.7 27.3) (width 0.6) (layer F.Cu) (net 7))
 (segment (start 7 30) (end 9 28) (width 1) (layer B.Cu) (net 7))
 (segment (start 7 30) (end 4 30) (width 1) (layer B.Cu) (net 7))
 (segment (start 10.04 26.96) (end 10.04 13.46) (width 1) (layer B.Cu) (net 7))
 (segment (start 9 28) (end 10.04 26.96) (width 1) (layer B.Cu) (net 7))
 (segment (start 6.54 4) (end 6.54 5.54) (width 1) (layer B.Cu) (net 7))
 (segment (start 10.04 9.04) (end 10.04 13.46) (width 1) (layer B.Cu) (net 7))
 (segment (start 6.54 5.54) (end 10.04 9.04) (width 1) (layer B.Cu) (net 7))
 (segment (start 11.905 31.595) (end 12.25 31.25) (width 0.6) (layer F.Cu) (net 6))
 (segment (start 9.475 31.595) (end 11.905 31.595) (width 0.6) (layer F.Cu) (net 6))
 (segment (start 12.5 31) (end 12.25 31.25) (width 0.6) (layer F.Cu) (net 6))
 (segment (start 12.5 28.25) (end 12.5 31) (width 0.6) (layer F.Cu) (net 6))
 (segment (start 13.31 18.69) (end 15 17) (width 0.6) (layer F.Cu) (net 16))
 (segment (start 13.31 20.975) (end 13.31 19.69) (width 0.6) (layer F.Cu) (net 16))
 (segment (start 15 17) (end 15 9) (width 0.6) (layer F.Cu) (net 16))
 (segment (start 10 4) (end 9.08 4) (width 0.6) (layer F.Cu) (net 16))
 (segment (start 15 9) (end 10 4) (width 0.6) (layer F.Cu) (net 16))
 (segment (start 12.185 34.135) (end 12.25 34.2) (width 0.6) (layer F.Cu) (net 10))
 (segment (start 9.475 34.135) (end 12.185 34.135) (width 0.6) (layer F.Cu) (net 10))
 (segment (start 14.3875 34.2) (end 14.5875 34) (width 0.6) (layer F.Cu) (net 10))
 (segment (start 12.25 34.2) (end 14.3875 34.2) (width 0.6) (layer F.Cu) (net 10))
 (segment (start 10.77 16.025) (end 10.77 17.73) (width 0.6) (layer F.Cu) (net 3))
 (segment (start 10.77 17.73) (end 10 18.5) (width 0.6) (layer F.Cu) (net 3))
 (via (at 7 18.5) (size 1.2) (drill 0.6) (layers F.Cu B.Cu) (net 3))
 (segment (start 10 18.5) (end 7 18.5) (width 0.6) (layer F.Cu) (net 3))
 (segment (start 5.42 20.08) (end 7 18.5) (width 0.6) (layer B.Cu) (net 3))
 (segment (start 3.5 20.08) (end 5.42 20.08) (width 0.6) (layer B.Cu) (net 3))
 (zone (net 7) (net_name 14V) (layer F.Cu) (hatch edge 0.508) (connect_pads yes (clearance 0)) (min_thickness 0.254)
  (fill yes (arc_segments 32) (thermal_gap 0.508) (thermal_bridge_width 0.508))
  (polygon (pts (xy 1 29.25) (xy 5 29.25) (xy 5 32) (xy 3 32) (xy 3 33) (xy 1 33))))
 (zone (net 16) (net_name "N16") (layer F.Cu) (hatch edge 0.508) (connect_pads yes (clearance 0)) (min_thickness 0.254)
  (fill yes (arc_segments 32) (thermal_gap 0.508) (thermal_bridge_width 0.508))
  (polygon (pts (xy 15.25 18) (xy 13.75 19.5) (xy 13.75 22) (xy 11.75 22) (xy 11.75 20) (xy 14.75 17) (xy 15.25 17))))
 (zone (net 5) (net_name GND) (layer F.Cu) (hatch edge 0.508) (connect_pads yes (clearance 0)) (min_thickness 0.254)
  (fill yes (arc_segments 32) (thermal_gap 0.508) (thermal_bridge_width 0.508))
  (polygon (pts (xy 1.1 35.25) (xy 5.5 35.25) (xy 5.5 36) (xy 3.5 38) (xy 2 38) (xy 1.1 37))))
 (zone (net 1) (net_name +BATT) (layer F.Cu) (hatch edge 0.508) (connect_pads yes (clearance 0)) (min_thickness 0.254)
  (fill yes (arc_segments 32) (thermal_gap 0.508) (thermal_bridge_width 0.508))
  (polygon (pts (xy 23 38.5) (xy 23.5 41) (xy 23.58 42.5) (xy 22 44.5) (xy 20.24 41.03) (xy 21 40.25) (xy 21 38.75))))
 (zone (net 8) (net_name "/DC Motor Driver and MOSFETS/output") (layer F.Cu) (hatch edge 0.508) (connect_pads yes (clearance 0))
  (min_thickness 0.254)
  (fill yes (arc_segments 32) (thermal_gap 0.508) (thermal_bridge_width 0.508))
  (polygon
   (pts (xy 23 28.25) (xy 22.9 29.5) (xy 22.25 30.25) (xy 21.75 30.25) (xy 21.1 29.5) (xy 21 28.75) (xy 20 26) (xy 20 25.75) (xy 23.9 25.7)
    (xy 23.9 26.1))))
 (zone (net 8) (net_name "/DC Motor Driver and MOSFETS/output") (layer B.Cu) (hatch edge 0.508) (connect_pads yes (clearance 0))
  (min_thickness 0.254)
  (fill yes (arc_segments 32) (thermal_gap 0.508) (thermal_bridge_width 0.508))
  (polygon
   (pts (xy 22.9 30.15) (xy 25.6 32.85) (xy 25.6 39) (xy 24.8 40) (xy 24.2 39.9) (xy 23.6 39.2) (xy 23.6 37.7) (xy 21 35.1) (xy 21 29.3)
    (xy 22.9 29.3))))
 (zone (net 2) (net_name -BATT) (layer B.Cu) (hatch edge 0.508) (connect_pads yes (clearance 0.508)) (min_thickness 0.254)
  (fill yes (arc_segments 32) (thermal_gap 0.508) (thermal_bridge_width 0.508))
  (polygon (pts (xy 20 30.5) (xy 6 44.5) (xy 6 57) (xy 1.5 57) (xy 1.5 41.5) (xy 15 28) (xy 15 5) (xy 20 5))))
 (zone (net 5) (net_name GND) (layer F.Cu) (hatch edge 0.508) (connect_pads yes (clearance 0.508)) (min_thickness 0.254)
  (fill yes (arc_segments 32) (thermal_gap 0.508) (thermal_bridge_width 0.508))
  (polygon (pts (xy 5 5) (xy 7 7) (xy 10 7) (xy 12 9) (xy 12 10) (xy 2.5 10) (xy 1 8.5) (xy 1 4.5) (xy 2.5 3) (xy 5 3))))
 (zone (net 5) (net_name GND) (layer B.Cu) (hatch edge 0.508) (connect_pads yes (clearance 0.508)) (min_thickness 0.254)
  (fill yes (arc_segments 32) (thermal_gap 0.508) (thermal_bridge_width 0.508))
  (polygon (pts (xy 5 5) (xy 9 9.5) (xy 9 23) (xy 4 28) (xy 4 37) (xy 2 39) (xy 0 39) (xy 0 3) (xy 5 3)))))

